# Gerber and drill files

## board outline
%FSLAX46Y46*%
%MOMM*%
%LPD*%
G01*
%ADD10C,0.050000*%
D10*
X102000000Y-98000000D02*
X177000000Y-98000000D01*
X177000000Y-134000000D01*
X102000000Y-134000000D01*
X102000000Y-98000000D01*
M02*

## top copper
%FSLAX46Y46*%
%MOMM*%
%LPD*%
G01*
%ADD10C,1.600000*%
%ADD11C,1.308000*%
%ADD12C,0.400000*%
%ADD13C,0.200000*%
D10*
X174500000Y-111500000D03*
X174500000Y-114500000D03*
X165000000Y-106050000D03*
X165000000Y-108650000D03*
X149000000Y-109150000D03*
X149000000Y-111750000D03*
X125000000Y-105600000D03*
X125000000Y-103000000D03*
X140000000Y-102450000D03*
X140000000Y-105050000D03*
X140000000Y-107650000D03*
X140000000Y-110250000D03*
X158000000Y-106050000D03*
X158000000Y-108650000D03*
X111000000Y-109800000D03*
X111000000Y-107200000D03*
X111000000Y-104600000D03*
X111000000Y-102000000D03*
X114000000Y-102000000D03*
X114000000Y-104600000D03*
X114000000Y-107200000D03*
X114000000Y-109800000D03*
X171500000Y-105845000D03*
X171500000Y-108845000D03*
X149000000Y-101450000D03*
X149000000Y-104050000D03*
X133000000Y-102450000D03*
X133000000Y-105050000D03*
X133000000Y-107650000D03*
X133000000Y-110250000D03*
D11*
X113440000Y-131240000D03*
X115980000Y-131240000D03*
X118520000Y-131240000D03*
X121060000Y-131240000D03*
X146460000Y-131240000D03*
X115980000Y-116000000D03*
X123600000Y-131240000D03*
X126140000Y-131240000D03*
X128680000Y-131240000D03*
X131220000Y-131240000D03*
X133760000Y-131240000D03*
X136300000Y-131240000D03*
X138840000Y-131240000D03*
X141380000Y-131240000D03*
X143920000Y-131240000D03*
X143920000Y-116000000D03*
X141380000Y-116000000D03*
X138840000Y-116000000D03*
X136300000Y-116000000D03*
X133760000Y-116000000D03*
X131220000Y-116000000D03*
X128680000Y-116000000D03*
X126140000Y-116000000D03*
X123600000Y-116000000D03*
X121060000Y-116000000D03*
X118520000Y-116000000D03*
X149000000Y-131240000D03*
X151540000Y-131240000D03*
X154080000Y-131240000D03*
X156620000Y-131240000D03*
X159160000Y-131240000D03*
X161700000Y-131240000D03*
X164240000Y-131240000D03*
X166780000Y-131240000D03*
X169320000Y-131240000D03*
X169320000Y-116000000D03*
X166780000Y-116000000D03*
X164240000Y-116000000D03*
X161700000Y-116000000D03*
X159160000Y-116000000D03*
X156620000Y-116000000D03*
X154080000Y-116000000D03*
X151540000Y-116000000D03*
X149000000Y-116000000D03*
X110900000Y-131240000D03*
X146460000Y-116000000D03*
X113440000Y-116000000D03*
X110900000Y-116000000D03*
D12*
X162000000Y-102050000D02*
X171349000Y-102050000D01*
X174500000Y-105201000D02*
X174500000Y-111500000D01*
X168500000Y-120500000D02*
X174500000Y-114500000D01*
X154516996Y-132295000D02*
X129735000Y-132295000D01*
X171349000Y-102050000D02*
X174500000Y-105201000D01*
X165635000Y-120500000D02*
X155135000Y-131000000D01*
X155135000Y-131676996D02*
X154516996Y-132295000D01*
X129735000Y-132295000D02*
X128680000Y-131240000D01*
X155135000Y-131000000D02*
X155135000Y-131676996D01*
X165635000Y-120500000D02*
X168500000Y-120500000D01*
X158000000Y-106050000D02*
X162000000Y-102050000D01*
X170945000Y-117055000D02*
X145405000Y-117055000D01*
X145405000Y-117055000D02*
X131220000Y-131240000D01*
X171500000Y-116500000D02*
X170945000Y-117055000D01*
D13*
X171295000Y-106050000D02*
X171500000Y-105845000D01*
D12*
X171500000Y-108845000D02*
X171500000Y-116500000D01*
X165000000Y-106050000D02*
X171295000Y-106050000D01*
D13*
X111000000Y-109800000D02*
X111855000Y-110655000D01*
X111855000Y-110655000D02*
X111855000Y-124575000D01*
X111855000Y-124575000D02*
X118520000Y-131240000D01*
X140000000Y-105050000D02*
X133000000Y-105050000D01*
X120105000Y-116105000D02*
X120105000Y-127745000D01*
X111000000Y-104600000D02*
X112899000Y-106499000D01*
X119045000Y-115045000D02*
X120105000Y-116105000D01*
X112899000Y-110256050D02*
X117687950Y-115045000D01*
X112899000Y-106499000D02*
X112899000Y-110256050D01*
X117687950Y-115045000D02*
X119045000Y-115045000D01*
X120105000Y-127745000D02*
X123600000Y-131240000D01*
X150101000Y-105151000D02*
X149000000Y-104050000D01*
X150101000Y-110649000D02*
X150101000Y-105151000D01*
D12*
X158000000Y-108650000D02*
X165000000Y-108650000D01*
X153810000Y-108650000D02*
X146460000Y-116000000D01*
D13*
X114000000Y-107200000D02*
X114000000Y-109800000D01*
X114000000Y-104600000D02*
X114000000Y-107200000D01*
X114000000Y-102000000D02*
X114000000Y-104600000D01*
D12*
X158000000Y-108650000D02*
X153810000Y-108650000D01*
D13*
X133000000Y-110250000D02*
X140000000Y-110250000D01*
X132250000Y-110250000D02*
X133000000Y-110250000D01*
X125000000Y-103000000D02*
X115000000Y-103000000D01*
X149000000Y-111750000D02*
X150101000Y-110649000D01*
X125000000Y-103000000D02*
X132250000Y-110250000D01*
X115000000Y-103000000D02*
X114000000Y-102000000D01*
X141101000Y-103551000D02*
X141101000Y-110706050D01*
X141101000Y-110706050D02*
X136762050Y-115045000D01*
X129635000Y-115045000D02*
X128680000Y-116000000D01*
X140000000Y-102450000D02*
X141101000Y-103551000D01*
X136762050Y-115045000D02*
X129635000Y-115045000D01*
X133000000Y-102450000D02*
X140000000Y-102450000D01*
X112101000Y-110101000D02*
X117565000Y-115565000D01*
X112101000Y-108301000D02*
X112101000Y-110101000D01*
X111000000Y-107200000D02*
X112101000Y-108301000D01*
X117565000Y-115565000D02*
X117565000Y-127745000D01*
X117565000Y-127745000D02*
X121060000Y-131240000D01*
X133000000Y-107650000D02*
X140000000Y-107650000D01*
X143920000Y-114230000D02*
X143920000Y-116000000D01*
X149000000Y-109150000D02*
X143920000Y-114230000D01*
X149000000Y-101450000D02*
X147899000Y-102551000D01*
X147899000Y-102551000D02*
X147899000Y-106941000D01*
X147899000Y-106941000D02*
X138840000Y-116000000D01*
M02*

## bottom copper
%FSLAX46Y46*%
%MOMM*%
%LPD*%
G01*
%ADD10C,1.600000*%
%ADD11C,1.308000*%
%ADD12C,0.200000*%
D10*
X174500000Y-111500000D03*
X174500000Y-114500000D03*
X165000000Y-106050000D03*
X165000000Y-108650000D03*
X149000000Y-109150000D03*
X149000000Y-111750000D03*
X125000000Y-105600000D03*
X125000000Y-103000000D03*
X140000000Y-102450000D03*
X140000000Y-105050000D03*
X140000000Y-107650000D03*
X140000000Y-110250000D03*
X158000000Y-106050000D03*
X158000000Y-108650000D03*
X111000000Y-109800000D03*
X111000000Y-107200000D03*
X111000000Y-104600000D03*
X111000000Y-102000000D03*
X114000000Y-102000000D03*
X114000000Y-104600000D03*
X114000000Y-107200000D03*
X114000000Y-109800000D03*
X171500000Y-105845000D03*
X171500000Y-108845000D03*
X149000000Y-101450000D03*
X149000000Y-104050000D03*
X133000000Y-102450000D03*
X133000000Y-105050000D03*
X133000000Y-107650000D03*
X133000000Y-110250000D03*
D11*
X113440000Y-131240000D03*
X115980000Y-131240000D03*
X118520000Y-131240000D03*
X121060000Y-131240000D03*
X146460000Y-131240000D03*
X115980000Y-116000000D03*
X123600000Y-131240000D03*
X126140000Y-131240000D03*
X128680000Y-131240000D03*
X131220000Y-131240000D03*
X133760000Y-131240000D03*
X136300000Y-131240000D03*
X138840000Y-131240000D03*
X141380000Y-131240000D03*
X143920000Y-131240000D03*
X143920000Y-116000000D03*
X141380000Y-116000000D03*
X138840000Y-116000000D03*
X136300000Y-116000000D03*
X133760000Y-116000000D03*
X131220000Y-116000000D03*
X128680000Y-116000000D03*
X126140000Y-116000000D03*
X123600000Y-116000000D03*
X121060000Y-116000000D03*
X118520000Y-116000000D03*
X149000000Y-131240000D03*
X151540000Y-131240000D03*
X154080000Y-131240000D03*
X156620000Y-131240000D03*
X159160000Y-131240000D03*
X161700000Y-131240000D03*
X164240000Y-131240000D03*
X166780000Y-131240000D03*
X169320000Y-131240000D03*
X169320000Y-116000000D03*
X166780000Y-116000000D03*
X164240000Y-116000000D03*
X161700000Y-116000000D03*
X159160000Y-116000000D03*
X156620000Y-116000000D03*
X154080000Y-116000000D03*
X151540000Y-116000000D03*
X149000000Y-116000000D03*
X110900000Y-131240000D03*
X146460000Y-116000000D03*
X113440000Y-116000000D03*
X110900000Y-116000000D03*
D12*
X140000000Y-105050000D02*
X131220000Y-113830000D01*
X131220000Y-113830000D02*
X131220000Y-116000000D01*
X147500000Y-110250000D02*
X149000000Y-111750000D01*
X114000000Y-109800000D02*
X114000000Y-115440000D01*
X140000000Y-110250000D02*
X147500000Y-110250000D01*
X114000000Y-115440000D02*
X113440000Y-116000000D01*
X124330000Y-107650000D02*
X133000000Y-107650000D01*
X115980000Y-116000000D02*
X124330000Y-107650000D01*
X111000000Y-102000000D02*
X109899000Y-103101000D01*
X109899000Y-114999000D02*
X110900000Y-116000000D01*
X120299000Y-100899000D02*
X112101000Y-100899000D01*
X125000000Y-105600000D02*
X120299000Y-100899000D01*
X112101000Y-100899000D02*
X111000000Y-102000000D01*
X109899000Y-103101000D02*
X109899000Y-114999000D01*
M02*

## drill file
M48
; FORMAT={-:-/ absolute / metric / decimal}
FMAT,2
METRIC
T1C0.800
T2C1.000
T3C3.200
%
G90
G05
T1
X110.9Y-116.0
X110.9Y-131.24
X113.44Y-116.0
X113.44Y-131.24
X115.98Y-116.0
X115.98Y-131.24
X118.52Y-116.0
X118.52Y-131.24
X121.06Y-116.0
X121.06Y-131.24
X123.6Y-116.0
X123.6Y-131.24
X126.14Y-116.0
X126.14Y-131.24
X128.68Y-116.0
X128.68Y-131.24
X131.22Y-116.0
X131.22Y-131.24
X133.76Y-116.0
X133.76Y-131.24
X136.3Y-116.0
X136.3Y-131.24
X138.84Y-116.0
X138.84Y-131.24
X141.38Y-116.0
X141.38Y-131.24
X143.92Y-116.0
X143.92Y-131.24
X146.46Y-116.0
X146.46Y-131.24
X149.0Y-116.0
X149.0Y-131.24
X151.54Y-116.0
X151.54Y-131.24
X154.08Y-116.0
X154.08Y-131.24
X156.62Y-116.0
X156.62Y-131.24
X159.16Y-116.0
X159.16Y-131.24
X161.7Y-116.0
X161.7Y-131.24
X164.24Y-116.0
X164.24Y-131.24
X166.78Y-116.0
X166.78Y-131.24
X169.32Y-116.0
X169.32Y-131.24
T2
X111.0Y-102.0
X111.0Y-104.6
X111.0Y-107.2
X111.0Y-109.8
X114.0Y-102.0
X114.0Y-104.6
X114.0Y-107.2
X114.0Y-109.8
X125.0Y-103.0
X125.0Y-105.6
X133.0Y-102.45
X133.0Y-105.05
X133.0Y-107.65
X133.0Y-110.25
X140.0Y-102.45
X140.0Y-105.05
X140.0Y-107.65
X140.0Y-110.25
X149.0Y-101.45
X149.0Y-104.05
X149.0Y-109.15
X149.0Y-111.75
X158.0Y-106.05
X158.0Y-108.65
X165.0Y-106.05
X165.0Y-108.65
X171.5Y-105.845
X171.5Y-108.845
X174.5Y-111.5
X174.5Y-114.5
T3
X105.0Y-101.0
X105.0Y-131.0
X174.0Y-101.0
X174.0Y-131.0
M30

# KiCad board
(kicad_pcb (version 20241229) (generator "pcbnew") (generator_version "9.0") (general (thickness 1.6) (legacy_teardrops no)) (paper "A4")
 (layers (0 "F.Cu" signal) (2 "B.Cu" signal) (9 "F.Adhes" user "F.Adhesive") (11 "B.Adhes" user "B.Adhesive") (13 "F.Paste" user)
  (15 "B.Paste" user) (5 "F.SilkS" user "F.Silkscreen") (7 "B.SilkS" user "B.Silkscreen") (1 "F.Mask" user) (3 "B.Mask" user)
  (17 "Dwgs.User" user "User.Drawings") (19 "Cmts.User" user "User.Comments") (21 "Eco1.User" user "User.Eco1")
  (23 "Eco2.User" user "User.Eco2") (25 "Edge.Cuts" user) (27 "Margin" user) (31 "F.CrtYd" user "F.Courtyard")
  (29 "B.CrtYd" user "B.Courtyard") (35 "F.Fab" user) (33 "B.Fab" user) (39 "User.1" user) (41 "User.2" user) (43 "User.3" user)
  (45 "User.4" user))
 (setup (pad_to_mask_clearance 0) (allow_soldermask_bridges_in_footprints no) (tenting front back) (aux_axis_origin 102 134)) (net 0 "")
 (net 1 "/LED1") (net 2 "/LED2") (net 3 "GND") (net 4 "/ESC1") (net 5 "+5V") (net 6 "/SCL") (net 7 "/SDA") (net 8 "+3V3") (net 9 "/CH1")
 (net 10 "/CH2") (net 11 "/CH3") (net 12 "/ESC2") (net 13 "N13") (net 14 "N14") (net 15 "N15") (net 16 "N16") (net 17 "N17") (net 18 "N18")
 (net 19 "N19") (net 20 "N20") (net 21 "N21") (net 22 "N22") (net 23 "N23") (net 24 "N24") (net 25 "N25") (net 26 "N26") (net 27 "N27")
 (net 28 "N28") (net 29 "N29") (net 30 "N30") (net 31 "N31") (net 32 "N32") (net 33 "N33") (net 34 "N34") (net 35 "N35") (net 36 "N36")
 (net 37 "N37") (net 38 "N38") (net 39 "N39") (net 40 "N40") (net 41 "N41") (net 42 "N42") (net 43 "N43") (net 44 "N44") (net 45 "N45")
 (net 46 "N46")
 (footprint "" (layer "F.Cu") (at 174 101)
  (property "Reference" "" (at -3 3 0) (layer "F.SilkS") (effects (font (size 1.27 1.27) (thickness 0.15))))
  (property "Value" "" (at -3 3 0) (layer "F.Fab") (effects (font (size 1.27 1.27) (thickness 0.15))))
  (pad "" np_thru_hole circle (at 0 0) (size 3.2 3.2) (drill 3.2) (layers "*.Cu" "*.Mask")))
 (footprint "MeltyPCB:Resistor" (layer "F.Cu") (at 176 113 -90)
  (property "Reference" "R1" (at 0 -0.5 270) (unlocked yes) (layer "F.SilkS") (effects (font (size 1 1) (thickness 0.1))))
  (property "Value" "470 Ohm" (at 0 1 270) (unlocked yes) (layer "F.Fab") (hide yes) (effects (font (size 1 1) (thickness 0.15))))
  (pad "1" thru_hole circle (at -1.5 1.5 270) (size 1.6 1.6) (drill 1) (layers "*.Cu" "*.Mask") (remove_unused_layers no) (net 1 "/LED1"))
  (pad "2" thru_hole circle (at 1.5 1.5 270) (size 1.6 1.6) (drill 1) (layers "*.Cu" "*.Mask") (remove_unused_layers no) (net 1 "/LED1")))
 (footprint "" (layer "F.Cu") (at 174 131)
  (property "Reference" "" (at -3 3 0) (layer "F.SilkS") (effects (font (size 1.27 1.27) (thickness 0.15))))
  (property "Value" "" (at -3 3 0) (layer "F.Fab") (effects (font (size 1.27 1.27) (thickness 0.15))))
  (pad "" np_thru_hole circle (at 0 0) (size 3.2 3.2) (drill 3.2) (layers "*.Cu" "*.Mask")))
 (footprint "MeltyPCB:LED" (layer "F.Cu") (at 165 104.05)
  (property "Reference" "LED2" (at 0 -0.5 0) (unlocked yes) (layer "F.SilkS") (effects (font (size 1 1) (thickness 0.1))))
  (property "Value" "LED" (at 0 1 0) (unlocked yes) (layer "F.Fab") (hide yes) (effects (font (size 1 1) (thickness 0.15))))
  (pad "1" thru_hole circle (at 0 2) (size 1.6 1.6) (drill 1) (layers "*.Cu" "*.Mask") (remove_unused_layers no) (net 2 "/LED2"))
  (pad "2" thru_hole circle (at 0 4.6) (size 1.6 1.6) (drill 1) (layers "*.Cu" "*.Mask") (remove_unused_layers no) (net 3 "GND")))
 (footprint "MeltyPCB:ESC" (layer "F.Cu") (at 149 107.25)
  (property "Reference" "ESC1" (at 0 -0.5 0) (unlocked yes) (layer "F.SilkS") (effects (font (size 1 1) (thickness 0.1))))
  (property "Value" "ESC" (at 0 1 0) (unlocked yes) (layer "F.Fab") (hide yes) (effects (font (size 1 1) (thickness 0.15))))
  (pad "1" thru_hole circle (at 0 1.9) (size 1.6 1.6) (drill 1) (layers "*.Cu" "*.Mask") (remove_unused_layers no) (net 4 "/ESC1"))
  (pad "2" thru_hole circle (at 0 4.5) (size 1.6 1.6) (drill 1) (layers "*.Cu" "*.Mask") (remove_unused_layers no) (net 3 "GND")))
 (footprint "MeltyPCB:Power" (layer "F.Cu") (at 125 107.4 180)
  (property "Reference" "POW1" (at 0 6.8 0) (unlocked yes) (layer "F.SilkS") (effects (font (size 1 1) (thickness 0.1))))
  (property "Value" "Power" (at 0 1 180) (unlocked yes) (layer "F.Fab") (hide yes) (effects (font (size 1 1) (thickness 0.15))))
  (pad "1" thru_hole circle (at 0 1.8 180) (size 1.6 1.6) (drill 1) (layers "*.Cu" "*.Mask") (remove_unused_layers no) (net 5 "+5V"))
  (pad "2" thru_hole circle (at 0 4.4 180) (size 1.6 1.6) (drill 1) (layers "*.Cu" "*.Mask") (remove_unused_layers no) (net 3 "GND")))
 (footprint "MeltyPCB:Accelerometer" (layer "F.Cu") (at 140 100.45)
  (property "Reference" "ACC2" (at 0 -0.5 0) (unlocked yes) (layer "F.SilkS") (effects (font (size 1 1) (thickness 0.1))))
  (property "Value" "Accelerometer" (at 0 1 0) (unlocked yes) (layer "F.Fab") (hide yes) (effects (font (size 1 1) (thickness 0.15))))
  (pad "1" thru_hole circle (at 0 2) (size 1.6 1.6) (drill 1) (layers "*.Cu" "*.Mask") (remove_unused_layers no) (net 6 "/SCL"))
  (pad "2" thru_hole circle (at 0 4.6) (size 1.6 1.6) (drill 1) (layers "*.Cu" "*.Mask") (remove_unused_layers no) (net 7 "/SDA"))
  (pad "3" thru_hole circle (at 0 7.2) (size 1.6 1.6) (drill 1) (layers "*.Cu" "*.Mask") (remove_unused_layers no) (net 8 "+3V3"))
  (pad "4" thru_hole circle (at 0 9.8) (size 1.6 1.6) (drill 1) (layers "*.Cu" "*.Mask") (remove_unused_layers no) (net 3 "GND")))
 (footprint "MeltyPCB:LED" (layer "F.Cu") (at 158 104.05)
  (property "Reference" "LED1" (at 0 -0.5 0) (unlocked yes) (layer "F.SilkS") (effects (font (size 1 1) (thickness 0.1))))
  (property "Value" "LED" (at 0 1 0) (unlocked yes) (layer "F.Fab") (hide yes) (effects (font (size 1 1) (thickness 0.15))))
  (pad "1" thru_hole circle (at 0 2) (size 1.6 1.6) (drill 1) (layers "*.Cu" "*.Mask") (remove_unused_layers no) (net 1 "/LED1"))
  (pad "2" thru_hole circle (at 0 4.6) (size 1.6 1.6) (drill 1) (layers "*.Cu" "*.Mask") (remove_unused_layers no) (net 3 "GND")))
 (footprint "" (layer "F.Cu") (at 105 101)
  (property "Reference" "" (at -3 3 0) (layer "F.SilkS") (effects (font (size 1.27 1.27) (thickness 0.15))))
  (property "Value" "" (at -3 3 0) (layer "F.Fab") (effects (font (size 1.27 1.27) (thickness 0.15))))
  (pad "" np_thru_hole circle (at 0 0) (size 3.2 3.2) (drill 3.2) (layers "*.Cu" "*.Mask")))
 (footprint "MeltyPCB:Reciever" (layer "F.Cu") (at 112.5 111.3 180)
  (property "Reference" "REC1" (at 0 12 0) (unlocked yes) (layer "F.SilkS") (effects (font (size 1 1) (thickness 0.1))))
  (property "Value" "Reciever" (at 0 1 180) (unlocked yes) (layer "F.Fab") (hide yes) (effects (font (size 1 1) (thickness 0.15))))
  (pad "1" thru_hole circle (at 1.5 1.5 180) (size 1.6 1.6) (drill 1) (layers "*.Cu" "*.Mask") (remove_unused_layers no) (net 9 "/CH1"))
  (pad "2" thru_hole circle (at 1.5 4.1 180) (size 1.6 1.6) (drill 1) (layers "*.Cu" "*.Mask") (remove_unused_layers no) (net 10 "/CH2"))
  (pad "3" thru_hole circle (at 1.5 6.7 180) (size 1.6 1.6) (drill 1) (layers "*.Cu" "*.Mask") (remove_unused_layers no) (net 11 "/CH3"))
  (pad "4" thru_hole circle (at 1.5 9.3 180) (size 1.6 1.6) (drill 1) (layers "*.Cu" "*.Mask") (remove_unused_layers no) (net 5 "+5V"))
  (pad "5" thru_hole circle (at -1.5 9.3 180) (size 1.6 1.6) (drill 1) (layers "*.Cu" "*.Mask") (remove_unused_layers no) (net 3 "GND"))
  (pad "6" thru_hole circle (at -1.5 6.7 180) (size 1.6 1.6) (drill 1) (layers "*.Cu" "*.Mask") (remove_unused_layers no) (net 3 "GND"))
  (pad "7" thru_hole circle (at -1.5 4.1 180) (size 1.6 1.6) (drill 1) (layers "*.Cu" "*.Mask") (remove_unused_layers no) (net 3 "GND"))
  (pad "8" thru_hole circle (at -1.5 1.5 180) (size 1.6 1.6) (drill 1) (layers "*.Cu" "*.Mask") (remove_unused_layers no) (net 3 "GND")))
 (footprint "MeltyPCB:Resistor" (layer "F.Cu") (at 173 107.345 -90)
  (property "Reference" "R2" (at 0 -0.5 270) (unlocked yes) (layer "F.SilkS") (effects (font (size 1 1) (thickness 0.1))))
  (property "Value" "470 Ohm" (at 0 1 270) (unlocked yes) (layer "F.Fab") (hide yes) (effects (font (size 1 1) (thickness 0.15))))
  (pad "1" thru_hole circle (at -1.5 1.5 270) (size 1.6 1.6) (drill 1) (layers "*.Cu" "*.Mask") (remove_unused_layers no) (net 2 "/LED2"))
  (pad "2" thru_hole circle (at 1.5 1.5 270) (size 1.6 1.6) (drill 1) (layers "*.Cu" "*.Mask") (remove_unused_layers no) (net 2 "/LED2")))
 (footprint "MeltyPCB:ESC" (layer "F.Cu") (at 149 99.55)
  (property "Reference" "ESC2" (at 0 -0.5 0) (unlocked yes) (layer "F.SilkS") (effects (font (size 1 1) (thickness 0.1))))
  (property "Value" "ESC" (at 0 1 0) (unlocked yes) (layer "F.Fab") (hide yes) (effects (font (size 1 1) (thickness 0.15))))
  (pad "1" thru_hole circle (at 0 1.9) (size 1.6 1.6) (drill 1) (layers "*.Cu" "*.Mask") (remove_unused_layers no) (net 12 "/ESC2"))
  (pad "2" thru_hole circle (at 0 4.5) (size 1.6 1.6) (drill 1) (layers "*.Cu" "*.Mask") (remove_unused_layers no) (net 3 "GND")))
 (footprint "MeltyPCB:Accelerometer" (layer "F.Cu") (at 133 100.45)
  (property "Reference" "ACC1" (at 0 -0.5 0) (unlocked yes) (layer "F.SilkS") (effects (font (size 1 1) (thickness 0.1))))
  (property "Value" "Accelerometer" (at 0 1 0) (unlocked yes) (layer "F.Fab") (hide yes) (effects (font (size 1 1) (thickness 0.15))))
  (pad "1" thru_hole circle (at 0 2) (size 1.6 1.6) (drill 1) (layers "*.Cu" "*.Mask") (remove_unused_layers no) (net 6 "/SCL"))
  (pad "2" thru_hole circle (at 0 4.6) (size 1.6 1.6) (drill 1) (layers "*.Cu" "*.Mask") (remove_unused_layers no) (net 7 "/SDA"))
  (pad "3" thru_hole circle (at 0 7.2) (size 1.6 1.6) (drill 1) (layers "*.Cu" "*.Mask") (remove_unused_layers no) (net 8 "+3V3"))
  (pad "4" thru_hole circle (at 0 9.8) (size 1.6 1.6) (drill 1) (layers "*.Cu" "*.Mask") (remove_unused_layers no) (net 3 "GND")))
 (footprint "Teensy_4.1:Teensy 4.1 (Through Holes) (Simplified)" (layer "F.Cu") (at 140.11 123.62)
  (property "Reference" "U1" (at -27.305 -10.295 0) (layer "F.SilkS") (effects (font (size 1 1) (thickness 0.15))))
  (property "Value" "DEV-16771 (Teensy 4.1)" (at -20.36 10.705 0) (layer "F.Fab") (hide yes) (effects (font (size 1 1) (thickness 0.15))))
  (pad "0" thru_hole circle (at -26.67 7.62) (size 1.308 1.308) (drill 0.8) (layers "*.Cu" "*.Mask") (remove_unused_layers no)
   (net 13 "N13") (solder_mask_margin 0.102))
  (pad "1" thru_hole circle (at -24.13 7.62) (size 1.308 1.308) (drill 0.8) (layers "*.Cu" "*.Mask") (remove_unused_layers no)
   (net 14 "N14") (solder_mask_margin 0.102))
  (pad "2" thru_hole circle (at -21.59 7.62) (size 1.308 1.308) (drill 0.8) (layers "*.Cu" "*.Mask") (remove_unused_layers no)
   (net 9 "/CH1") (solder_mask_margin 0.102))
  (pad "3" thru_hole circle (at -19.05 7.62) (size 1.308 1.308) (drill 0.8) (layers "*.Cu" "*.Mask") (remove_unused_layers no)
   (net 10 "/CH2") (solder_mask_margin 0.102))
  (pad "3.3V_1" thru_hole circle (at 6.35 7.62) (size 1.308 1.308) (drill 0.8) (layers "*.Cu" "*.Mask") (remove_unused_layers no)
   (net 8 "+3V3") (solder_mask_margin 0.102))
  (pad "3.3V_2" thru_hole circle (at -24.13 -7.62) (size 1.308 1.308) (drill 0.8) (layers "*.Cu" "*.Mask") (remove_unused_layers no)
   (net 8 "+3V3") (solder_mask_margin 0.102))
  (pad "4" thru_hole circle (at -16.51 7.62) (size 1.308 1.308) (drill 0.8) (layers "*.Cu" "*.Mask") (remove_unused_layers no)
   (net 11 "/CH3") (solder_mask_margin 0.102))
  (pad "5" thru_hole circle (at -13.97 7.62) (size 1.308 1.308) (drill 0.8) (layers "*.Cu" "*.Mask") (remove_unused_layers no)
   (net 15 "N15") (solder_mask_margin 0.102))
  (pad "6" thru_hole circle (at -11.43 7.62) (size 1.308 1.308) (drill 0.8) (layers "*.Cu" "*.Mask") (remove_unused_layers no)
   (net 1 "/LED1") (solder_mask_margin 0.102))
  (pad "7" thru_hole circle (at -8.89 7.62) (size 1.308 1.308) (drill 0.8) (layers "*.Cu" "*.Mask") (remove_unused_layers no)
   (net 2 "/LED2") (solder_mask_margin 0.102))
  (pad "8" thru_hole circle (at -6.35 7.62) (size 1.308 1.308) (drill 0.8) (layers "*.Cu" "*.Mask") (remove_unused_layers no) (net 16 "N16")
   (solder_mask_margin 0.102))
  (pad "9" thru_hole circle (at -3.81 7.62) (size 1.308 1.308) (drill 0.8) (layers "*.Cu" "*.Mask") (remove_unused_layers no) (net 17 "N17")
   (solder_mask_margin 0.102))
  (pad "10" thru_hole circle (at -1.27 7.62) (size 1.308 1.308) (drill 0.8) (layers "*.Cu" "*.Mask") (remove_unused_layers no)
   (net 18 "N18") (solder_mask_margin 0.102))
  (pad "11" thru_hole circle (at 1.27 7.62) (size 1.308 1.308) (drill 0.8) (layers "*.Cu" "*.Mask") (remove_unused_layers no) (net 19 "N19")
   (solder_mask_margin 0.102))
  (pad "12" thru_hole circle (at 3.81 7.62) (size 1.308 1.308) (drill 0.8) (layers "*.Cu" "*.Mask") (remove_unused_layers no) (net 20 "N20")
   (solder_mask_margin 0.102))
  (pad "13" thru_hole circle (at 3.81 -7.62) (size 1.308 1.308) (drill 0.8) (layers "*.Cu" "*.Mask") (remove_unused_layers no)
   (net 4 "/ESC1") (solder_mask_margin 0.102))
  (pad "14" thru_hole circle (at 1.27 -7.62) (size 1.308 1.308) (drill 0.8) (layers "*.Cu" "*.Mask") (remove_unused_layers no)
   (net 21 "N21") (solder_mask_margin 0.102))
  (pad "15" thru_hole circle (at -1.27 -7.62) (size 1.308 1.308) (drill 0.8) (layers "*.Cu" "*.Mask") (remove_unused_layers no)
   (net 12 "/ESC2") (solder_mask_margin 0.102))
  (pad "16" thru_hole circle (at -3.81 -7.62) (size 1.308 1.308) (drill 0.8) (layers "*.Cu" "*.Mask") (remove_unused_layers no)
   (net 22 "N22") (solder_mask_margin 0.102))
  (pad "17" thru_hole circle (at -6.35 -7.62) (size 1.308 1.308) (drill 0.8) (layers "*.Cu" "*.Mask") (remove_unused_layers no)
   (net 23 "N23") (solder_mask_margin 0.102))
  (pad "18" thru_hole circle (at -8.89 -7.62) (size 1.308 1.308) (drill 0.8) (layers "*.Cu" "*.Mask") (remove_unused_layers no)
   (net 7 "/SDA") (solder_mask_margin 0.102))
  (pad "19" thru_hole circle (at -11.43 -7.62) (size 1.308 1.308) (drill 0.8) (layers "*.Cu" "*.Mask") (remove_unused_layers no)
   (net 6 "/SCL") (solder_mask_margin 0.102))
  (pad "20" thru_hole circle (at -13.97 -7.62) (size 1.308 1.308) (drill 0.8) (layers "*.Cu" "*.Mask") (remove_unused_layers no)
   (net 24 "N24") (solder_mask_margin 0.102))
  (pad "21" thru_hole circle (at -16.51 -7.62) (size 1.308 1.308) (drill 0.8) (layers "*.Cu" "*.Mask") (remove_unused_layers no)
   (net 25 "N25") (solder_mask_margin 0.102))
  (pad "22" thru_hole circle (at -19.05 -7.62) (size 1.308 1.308) (drill 0.8) (layers "*.Cu" "*.Mask") (remove_unused_layers no)
   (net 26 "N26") (solder_mask_margin 0.102))
  (pad "23" thru_hole circle (at -21.59 -7.62) (size 1.308 1.308) (drill 0.8) (layers "*.Cu" "*.Mask") (remove_unused_layers no)
   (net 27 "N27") (solder_mask_margin 0.102))
  (pad "24" thru_hole circle (at 8.89 7.62) (size 1.308 1.308) (drill 0.8) (layers "*.Cu" "*.Mask") (remove_unused_layers no) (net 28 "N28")
   (solder_mask_margin 0.102))
  (pad "25" thru_hole circle (at 11.43 7.62) (size 1.308 1.308) (drill 0.8) (layers "*.Cu" "*.Mask") (remove_unused_layers no)
   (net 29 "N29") (solder_mask_margin 0.102))
  (pad "26" thru_hole circle (at 13.97 7.62) (size 1.308 1.308) (drill 0.8) (layers "*.Cu" "*.Mask") (remove_unused_layers no)
   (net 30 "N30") (solder_mask_margin 0.102))
  (pad "27" thru_hole circle (at 16.51 7.62) (size 1.308 1.308) (drill 0.8) (layers "*.Cu" "*.Mask") (remove_unused_layers no)
   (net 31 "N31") (solder_mask_margin 0.102))
  (pad "28" thru_hole circle (at 19.05 7.62) (size 1.308 1.308) (drill 0.8) (layers "*.Cu" "*.Mask") (remove_unused_layers no)
   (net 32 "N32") (solder_mask_margin 0.102))
  (pad "29" thru_hole circle (at 21.59 7.62) (size 1.308 1.308) (drill 0.8) (layers "*.Cu" "*.Mask") (remove_unused_layers no)
   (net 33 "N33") (solder_mask_margin 0.102))
  (pad "30" thru_hole circle (at 24.13 7.62) (size 1.308 1.308) (drill 0.8) (layers "*.Cu" "*.Mask") (remove_unused_layers no)
   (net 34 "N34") (solder_mask_margin 0.102))
  (pad "31" thru_hole circle (at 26.67 7.62) (size 1.308 1.308) (drill 0.8) (layers "*.Cu" "*.Mask") (remove_unused_layers no)
   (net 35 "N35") (solder_mask_margin 0.102))
  (pad "32" thru_hole circle (at 29.21 7.62) (size 1.308 1.308) (drill 0.8) (layers "*.Cu" "*.Mask") (remove_unused_layers no)
   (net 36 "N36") (solder_mask_margin 0.102))
  (pad "33" thru_hole circle (at 29.21 -7.62) (size 1.308 1.308) (drill 0.8) (layers "*.Cu" "*.Mask") (remove_unused_layers no)
   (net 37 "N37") (solder_mask_margin 0.102))
  (pad "34" thru_hole circle (at 26.67 -7.62) (size 1.308 1.308) (drill 0.8) (layers "*.Cu" "*.Mask") (remove_unused_layers no)
   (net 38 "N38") (solder_mask_margin 0.102))
  (pad "35" thru_hole circle (at 24.13 -7.62) (size 1.308 1.308) (drill 0.8) (layers "*.Cu" "*.Mask") (remove_unused_layers no)
   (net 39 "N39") (solder_mask_margin 0.102))
  (pad "36" thru_hole circle (at 21.59 -7.62) (size 1.308 1.308) (drill 0.8) (layers "*.Cu" "*.Mask") (remove_unused_layers no)
   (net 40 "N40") (solder_mask_margin 0.102))
  (pad "37" thru_hole circle (at 19.05 -7.62) (size 1.308 1.308) (drill 0.8) (layers "*.Cu" "*.Mask") (remove_unused_layers no)
   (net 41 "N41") (solder_mask_margin 0.102))
  (pad "38" thru_hole circle (at 16.51 -7.62) (size 1.308 1.308) (drill 0.8) (layers "*.Cu" "*.Mask") (remove_unused_layers no)
   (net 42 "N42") (solder_mask_margin 0.102))
  (pad "39" thru_hole circle (at 13.97 -7.62) (size 1.308 1.308) (drill 0.8) (layers "*.Cu" "*.Mask") (remove_unused_layers no)
   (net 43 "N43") (solder_mask_margin 0.102))
  (pad "40" thru_hole circle (at 11.43 -7.62) (size 1.308 1.308) (drill 0.8) (layers "*.Cu" "*.Mask") (remove_unused_layers no)
   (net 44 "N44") (solder_mask_margin 0.102))
  (pad "41" thru_hole circle (at 8.89 -7.62) (size 1.308 1.308) (drill 0.8) (layers "*.Cu" "*.Mask") (remove_unused_layers no)
   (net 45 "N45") (solder_mask_margin 0.102))
  (pad "GND1" thru_hole circle (at -29.21 7.62) (size 1.308 1.308) (drill 0.8) (layers "*.Cu" "*.Mask") (remove_unused_layers no)
   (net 3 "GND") (solder_mask_margin 0.102))
  (pad "GND2" thru_hole circle (at 6.35 -7.62) (size 1.308 1.308) (drill 0.8) (layers "*.Cu" "*.Mask") (remove_unused_layers no)
   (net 3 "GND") (solder_mask_margin 0.102))
  (pad "GND3" thru_hole circle (at -26.67 -7.62) (size 1.308 1.308) (drill 0.8) (layers "*.Cu" "*.Mask") (remove_unused_layers no)
   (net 3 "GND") (solder_mask_margin 0.102))
  (pad "VIN" thru_hole circle (at -29.21 -7.62) (size 1.308 1.308) (drill 0.8) (layers "*.Cu" "*.Mask") (remove_unused_layers no)
   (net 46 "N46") (solder_mask_margin 0.102)))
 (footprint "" (layer "F.Cu") (at 105 131)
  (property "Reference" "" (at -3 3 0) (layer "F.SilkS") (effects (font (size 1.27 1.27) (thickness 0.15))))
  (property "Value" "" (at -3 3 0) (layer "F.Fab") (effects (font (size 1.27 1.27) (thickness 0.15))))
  (pad "" np_thru_hole circle (at 0 0) (size 3.2 3.2) (drill 3.2) (layers "*.Cu" "*.Mask")))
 (gr_rect (start 102 98) (end 177 134) (stroke (width 0.05) (type default)) (fill no) (layer "Edge.Cuts"))
 (segment (start 162 102.05) (end 171.349 102.05) (width 0.4) (layer "F.Cu") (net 1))
 (segment (start 174.5 105.201) (end 174.5 111.5) (width 0.4) (layer "F.Cu") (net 1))
 (segment (start 168.5 120.5) (end 174.5 114.5) (width 0.4) (layer "F.Cu") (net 1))
 (segment (start 154.516996 132.295) (end 129.735 132.295) (width 0.4) (layer "F.Cu") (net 1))
 (segment (start 171.349 102.05) (end 174.5 105.201) (width 0.4) (layer "F.Cu") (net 1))
 (segment (start 165.635 120.5) (end 155.135 131) (width 0.4) (layer "F.Cu") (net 1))
 (segment (start 155.135 131.676996) (end 154.516996 132.295) (width 0.4) (layer "F.Cu") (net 1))
 (segment (start 129.735 132.295) (end 128.68 131.24) (width 0.4) (layer "F.Cu") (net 1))
 (segment (start 155.135 131) (end 155.135 131.676996) (width 0.4) (layer "F.Cu") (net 1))
 (segment (start 165.635 120.5) (end 168.5 120.5) (width 0.4) (layer "F.Cu") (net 1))
 (segment (start 158 106.05) (end 162 102.05) (width 0.4) (layer "F.Cu") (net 1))
 (segment (start 170.945 117.055) (end 145.405 117.055) (width 0.4) (layer "F.Cu") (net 2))
 (segment (start 145.405 117.055) (end 131.22 131.24) (width 0.4) (layer "F.Cu") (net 2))
 (segment (start 171.5 116.5) (end 170.945 117.055) (width 0.4) (layer "F.Cu") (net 2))
 (segment (start 171.295 106.05) (end 171.5 105.845) (width 0.2) (layer "F.Cu") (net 2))
 (segment (start 171.5 108.845) (end 171.5 116.5) (width 0.4) (layer "F.Cu") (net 2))
 (segment (start 165 106.05) (end 171.295 106.05) (width 0.4) (layer "F.Cu") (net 2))
 (segment (start 111 109.8) (end 111.855 110.655) (width 0.2) (layer "F.Cu") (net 9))
 (segment (start 111.855 110.655) (end 111.855 124.575) (width 0.2) (layer "F.Cu") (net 9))
 (segment (start 111.855 124.575) (end 118.52 131.24) (width 0.2) (layer "F.Cu") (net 9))
 (segment (start 140 105.05) (end 133 105.05) (width 0.2) (layer "F.Cu") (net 7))
 (segment (start 140 105.05) (end 131.22 113.83) (width 0.2) (layer "B.Cu") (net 7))
 (segment (start 131.22 113.83) (end 131.22 116) (width 0.2) (layer "B.Cu") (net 7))
 (segment (start 120.105 116.105) (end 120.105 127.745) (width 0.2) (layer "F.Cu") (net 11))
 (segment (start 111 104.6) (end 112.899 106.499) (width 0.2) (layer "F.Cu") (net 11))
 (segment (start 119.045 115.045) (end 120.105 116.105) (width 0.2) (layer "F.Cu") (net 11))
 (segment (start 112.899 110.25605) (end 117.68795 115.045) (width 0.2) (layer "F.Cu") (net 11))
 (segment (start 112.899 106.499) (end 112.899 110.25605) (width 0.2) (layer "F.Cu") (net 11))
 (segment (start 117.68795 115.045) (end 119.045 115.045) (width 0.2) (layer "F.Cu") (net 11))
 (segment (start 120.105 127.745) (end 123.6 131.24) (width 0.2) (layer "F.Cu") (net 11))
 (segment (start 150.101 105.151) (end 149 104.05) (width 0.2) (layer "F.Cu") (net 3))
 (segment (start 150.101 110.649) (end 150.101 105.151) (width 0.2) (layer "F.Cu") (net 3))
 (segment (start 158 108.65) (end 165 108.65) (width 0.4) (layer "F.Cu") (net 3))
 (segment (start 153.81 108.65) (end 146.46 116) (width 0.4) (layer "F.Cu") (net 3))
 (segment (start 114 107.2) (end 114 109.8) (width 0.2) (layer "F.Cu") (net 3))
 (segment (start 114 104.6) (end 114 107.2) (width 0.2) (layer "F.Cu") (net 3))
 (segment (start 114 102) (end 114 104.6) (width 0.2) (layer "F.Cu") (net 3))
 (segment (start 158 108.65) (end 153.81 108.65) (width 0.4) (layer "F.Cu") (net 3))
 (segment (start 133 110.25) (end 140 110.25) (width 0.2) (layer "F.Cu") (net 3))
 (segment (start 132.25 110.25) (end 133 110.25) (width 0.2) (layer "F.Cu") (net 3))
 (segment (start 125 103) (end 115 103) (width 0.2) (layer "F.Cu") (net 3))
 (segment (start 149 111.75) (end 150.101 110.649) (width 0.2) (layer "F.Cu") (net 3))
 (segment (start 125 103) (end 132.25 110.25) (width 0.2) (layer "F.Cu") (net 3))
 (segment (start 115 103) (end 114 102) (width 0.2) (layer "F.Cu") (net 3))
 (segment (start 147.5 110.25) (end 149 111.75) (width 0.2) (layer "B.Cu") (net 3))
 (segment (start 114 109.8) (end 114 115.44) (width 0.2) (layer "B.Cu") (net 3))
 (segment (start 140 110.25) (end 147.5 110.25) (width 0.2) (layer "B.Cu") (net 3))
 (segment (start 114 115.44) (end 113.44 116) (width 0.2) (layer "B.Cu") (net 3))
 (segment (start 141.101 103.551) (end 141.101 110.70605) (width 0.2) (layer "F.Cu") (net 6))
 (segment (start 141.101 110.70605) (end 136.76205 115.045) (width 0.2) (layer "F.Cu") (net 6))
 (segment (start 129.635 115.045) (end 128.68 116) (width 0.2) (layer "F.Cu") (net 6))
 (segment (start 140 102.45) (end 141.101 103.551) (width 0.2) (layer "F.Cu") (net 6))
 (segment (start 136.76205 115.045) (end 129.635 115.045) (width 0.2) (layer "F.Cu") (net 6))
 (segment (start 133 102.45) (end 140 102.45) (width 0.2) (layer "F.Cu") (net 6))
 (segment (start 112.101 110.101) (end 117.565 115.565) (width 0.2) (layer "F.Cu") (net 10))
 (segment (start 112.101 108.301) (end 112.101 110.101) (width 0.2) (layer "F.Cu") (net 10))
 (segment (start 111 107.2) (end 112.101 108.301) (width 0.2) (layer "F.Cu") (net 10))
 (segment (start 117.565 115.565) (end 117.565 127.745) (width 0.2) (layer "F.Cu") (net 10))
 (segment (start 117.565 127.745) (end 121.06 131.24) (width 0.2) (layer "F.Cu") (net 10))
 (segment (start 133 107.65) (end 140 107.65) (width 0.2) (layer "F.Cu") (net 8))
 (segment (start 124.33 107.65) (end 133 107.65) (width 0.2) (layer "B.Cu") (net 8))
 (segment (start 115.98 116) (end 124.33 107.65) (width 0.2) (layer "B.Cu") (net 8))
 (segment (start 111 102) (end 109.899 103.101) (width 0.2) (layer "B.Cu") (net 5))
 (segment (start 109.899 114.999) (end 110.9 116) (width 0.2) (layer "B.Cu") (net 5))
 (segment (start 120.299 100.899) (end 112.101 100.899) (width 0.2) (layer "B.Cu") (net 5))
 (segment (start 125 105.6) (end 120.299 100.899) (width 0.2) (layer "B.Cu") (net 5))
 (segment (start 112.101 100.899) (end 111 102) (width 0.2) (layer "B.Cu") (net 5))
 (segment (start 109.899 103.101) (end 109.899 114.999) (width 0.2) (layer "B.Cu") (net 5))
 (segment (start 143.92 114.23) (end 143.92 116) (width 0.2) (layer "F.Cu") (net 4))
 (segment (start 149 109.15) (end 143.92 114.23) (width 0.2) (layer "F.Cu") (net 4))
 (segment (start 149 101.45) (end 147.899 102.551) (width 0.2) (layer "F.Cu") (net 12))
 (segment (start 147.899 102.551) (end 147.899 106.941) (width 0.2) (layer "F.Cu") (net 12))
 (segment (start 147.899 106.941) (end 138.84 116) (width 0.2) (layer "F.Cu") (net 12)))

